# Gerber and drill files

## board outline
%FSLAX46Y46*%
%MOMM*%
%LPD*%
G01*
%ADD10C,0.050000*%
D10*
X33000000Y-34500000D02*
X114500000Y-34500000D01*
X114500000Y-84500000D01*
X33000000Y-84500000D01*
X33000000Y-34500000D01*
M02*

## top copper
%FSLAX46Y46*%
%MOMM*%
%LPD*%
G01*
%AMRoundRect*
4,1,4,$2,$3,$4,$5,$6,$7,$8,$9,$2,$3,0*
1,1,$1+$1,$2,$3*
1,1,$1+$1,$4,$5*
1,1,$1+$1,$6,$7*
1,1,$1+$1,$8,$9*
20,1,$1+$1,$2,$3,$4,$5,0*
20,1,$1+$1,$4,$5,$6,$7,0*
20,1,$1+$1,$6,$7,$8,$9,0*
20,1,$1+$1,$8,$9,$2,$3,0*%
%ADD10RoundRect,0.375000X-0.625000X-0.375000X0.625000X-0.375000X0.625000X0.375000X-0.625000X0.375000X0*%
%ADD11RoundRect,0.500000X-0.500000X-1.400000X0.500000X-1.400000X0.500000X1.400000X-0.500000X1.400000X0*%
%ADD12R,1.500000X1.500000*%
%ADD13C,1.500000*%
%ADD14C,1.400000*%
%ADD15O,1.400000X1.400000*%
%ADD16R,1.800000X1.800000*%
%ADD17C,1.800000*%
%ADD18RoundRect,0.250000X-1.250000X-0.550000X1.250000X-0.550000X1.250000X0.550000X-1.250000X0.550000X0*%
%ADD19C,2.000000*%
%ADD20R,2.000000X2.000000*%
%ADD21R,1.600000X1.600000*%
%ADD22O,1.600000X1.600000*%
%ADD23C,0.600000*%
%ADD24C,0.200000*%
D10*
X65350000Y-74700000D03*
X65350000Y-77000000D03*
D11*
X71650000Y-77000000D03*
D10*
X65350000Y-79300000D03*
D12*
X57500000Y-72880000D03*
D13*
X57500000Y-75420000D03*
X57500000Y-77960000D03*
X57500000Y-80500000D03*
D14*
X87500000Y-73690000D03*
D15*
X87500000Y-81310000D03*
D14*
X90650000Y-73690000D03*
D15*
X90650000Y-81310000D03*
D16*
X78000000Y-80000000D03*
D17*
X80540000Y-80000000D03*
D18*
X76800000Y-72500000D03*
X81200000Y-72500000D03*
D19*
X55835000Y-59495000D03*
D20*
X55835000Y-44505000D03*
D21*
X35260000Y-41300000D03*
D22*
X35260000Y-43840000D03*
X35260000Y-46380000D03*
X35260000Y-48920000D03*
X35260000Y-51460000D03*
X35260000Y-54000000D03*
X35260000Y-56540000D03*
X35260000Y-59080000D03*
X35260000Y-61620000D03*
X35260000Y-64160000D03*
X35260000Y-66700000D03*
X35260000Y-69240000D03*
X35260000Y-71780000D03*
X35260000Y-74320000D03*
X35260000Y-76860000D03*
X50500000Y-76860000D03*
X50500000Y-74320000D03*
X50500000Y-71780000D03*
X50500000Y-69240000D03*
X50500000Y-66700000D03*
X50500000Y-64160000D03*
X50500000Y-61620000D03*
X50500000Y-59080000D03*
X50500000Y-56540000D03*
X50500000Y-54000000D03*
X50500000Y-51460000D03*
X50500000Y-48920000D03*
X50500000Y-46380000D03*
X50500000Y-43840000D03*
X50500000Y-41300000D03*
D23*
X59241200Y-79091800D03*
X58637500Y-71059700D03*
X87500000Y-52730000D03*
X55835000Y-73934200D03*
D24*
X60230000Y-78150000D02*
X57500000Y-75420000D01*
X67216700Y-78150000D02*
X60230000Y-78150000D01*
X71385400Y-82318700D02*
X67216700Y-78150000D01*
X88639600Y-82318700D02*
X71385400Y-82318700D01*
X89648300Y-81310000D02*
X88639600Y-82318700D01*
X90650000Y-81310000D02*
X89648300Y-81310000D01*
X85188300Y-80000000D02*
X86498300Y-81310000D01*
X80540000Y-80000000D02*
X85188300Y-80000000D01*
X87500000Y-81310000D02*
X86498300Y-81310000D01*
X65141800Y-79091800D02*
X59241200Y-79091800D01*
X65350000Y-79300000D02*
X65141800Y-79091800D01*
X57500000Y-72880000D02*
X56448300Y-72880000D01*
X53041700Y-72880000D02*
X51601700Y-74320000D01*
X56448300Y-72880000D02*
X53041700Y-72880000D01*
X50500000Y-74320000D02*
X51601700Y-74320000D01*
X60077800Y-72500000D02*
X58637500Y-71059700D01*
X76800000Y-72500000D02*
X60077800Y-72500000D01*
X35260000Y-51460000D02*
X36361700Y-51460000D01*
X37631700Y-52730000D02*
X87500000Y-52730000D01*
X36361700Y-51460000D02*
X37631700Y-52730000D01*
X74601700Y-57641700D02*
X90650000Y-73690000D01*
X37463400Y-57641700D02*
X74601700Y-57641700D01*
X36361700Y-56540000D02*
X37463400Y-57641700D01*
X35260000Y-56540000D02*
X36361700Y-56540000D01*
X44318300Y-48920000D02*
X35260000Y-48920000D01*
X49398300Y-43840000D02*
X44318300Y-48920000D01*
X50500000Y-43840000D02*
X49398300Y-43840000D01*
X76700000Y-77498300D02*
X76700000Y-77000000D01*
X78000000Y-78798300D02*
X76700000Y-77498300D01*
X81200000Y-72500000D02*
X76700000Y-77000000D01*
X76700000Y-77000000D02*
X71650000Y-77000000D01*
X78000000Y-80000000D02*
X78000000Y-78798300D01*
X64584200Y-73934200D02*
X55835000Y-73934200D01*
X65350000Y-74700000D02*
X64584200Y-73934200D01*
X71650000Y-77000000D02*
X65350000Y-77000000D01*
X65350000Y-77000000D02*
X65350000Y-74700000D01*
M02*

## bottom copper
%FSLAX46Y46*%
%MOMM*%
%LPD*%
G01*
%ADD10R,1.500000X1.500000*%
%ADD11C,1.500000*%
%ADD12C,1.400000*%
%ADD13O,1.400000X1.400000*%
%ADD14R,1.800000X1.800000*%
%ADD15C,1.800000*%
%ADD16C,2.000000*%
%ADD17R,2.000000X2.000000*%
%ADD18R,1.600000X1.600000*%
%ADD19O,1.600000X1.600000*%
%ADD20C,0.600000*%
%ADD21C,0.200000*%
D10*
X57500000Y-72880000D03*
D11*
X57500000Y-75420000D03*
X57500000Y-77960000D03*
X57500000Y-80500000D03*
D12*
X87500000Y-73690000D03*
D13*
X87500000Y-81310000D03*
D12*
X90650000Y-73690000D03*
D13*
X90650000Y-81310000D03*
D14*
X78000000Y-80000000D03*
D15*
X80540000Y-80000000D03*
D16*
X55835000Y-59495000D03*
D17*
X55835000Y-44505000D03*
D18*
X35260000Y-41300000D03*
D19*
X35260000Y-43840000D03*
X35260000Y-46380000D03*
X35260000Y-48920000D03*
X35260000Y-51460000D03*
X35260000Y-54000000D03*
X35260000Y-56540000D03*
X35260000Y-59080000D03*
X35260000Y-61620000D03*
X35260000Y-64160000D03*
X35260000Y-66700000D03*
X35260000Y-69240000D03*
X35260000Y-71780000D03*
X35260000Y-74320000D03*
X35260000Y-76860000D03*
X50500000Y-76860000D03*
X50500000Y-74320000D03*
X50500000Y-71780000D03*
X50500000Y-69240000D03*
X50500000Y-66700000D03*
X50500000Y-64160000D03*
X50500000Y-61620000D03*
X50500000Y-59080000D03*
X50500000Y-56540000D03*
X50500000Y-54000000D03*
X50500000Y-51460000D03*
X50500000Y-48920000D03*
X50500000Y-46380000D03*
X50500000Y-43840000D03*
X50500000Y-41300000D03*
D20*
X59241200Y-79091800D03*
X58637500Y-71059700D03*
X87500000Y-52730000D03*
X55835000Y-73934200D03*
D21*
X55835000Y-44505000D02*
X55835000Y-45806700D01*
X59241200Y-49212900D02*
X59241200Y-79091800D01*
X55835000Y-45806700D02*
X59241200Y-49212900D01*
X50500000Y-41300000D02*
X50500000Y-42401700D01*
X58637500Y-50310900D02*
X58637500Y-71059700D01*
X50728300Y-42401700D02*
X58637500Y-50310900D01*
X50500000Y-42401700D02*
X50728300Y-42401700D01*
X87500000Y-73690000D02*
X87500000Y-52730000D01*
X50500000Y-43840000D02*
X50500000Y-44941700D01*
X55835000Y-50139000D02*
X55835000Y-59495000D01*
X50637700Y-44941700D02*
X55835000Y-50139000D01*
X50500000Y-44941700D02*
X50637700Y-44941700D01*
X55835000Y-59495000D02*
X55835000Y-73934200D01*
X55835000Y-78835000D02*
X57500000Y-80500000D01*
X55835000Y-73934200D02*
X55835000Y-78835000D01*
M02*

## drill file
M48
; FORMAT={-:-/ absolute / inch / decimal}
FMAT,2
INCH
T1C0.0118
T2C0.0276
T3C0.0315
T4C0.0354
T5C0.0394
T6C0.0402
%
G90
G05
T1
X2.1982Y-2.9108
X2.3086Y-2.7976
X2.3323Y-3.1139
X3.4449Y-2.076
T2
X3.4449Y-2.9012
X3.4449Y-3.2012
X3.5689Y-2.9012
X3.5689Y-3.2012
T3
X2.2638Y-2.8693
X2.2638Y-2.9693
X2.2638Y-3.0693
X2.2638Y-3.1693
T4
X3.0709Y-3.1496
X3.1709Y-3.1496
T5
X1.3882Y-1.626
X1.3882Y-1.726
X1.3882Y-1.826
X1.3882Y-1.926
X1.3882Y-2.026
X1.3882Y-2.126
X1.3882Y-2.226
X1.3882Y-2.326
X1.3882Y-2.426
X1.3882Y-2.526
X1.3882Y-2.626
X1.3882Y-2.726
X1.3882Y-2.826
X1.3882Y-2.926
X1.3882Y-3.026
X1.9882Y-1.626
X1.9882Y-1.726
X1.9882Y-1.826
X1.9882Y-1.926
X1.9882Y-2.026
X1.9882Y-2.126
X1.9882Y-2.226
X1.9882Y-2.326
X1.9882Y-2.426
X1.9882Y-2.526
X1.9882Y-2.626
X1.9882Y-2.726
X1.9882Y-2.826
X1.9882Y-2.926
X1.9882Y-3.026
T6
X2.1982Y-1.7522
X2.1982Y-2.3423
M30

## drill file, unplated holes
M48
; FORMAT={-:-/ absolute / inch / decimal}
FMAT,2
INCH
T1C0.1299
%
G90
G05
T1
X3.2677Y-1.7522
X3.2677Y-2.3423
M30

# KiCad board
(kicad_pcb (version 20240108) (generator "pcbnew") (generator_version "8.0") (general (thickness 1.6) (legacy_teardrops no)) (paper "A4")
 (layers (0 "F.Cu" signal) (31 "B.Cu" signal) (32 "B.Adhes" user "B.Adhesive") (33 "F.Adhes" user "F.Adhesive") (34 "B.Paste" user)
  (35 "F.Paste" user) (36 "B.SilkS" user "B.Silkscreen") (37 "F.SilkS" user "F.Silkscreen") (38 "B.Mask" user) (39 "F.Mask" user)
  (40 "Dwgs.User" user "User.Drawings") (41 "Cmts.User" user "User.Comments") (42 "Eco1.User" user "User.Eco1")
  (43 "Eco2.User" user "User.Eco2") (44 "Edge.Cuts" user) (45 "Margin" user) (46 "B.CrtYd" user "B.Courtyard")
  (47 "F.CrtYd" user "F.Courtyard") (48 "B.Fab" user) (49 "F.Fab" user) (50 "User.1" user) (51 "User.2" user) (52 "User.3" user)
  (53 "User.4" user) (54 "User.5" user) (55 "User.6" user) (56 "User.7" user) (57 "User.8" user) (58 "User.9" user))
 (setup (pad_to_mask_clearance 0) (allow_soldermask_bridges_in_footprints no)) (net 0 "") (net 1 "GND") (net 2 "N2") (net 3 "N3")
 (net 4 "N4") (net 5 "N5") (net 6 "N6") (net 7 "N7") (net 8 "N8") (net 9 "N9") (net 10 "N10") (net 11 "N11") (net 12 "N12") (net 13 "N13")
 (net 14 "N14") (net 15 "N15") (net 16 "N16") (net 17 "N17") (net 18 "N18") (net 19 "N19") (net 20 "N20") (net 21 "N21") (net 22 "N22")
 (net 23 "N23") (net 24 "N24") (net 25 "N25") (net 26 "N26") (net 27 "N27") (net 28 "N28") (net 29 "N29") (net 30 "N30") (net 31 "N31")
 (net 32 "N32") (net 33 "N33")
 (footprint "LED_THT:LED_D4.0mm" (layer "F.Cu") (at 78 80)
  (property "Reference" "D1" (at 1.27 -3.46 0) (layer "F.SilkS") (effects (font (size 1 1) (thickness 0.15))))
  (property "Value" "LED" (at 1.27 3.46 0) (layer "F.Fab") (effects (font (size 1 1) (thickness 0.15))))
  (pad "1" thru_hole rect (at 0 0) (size 1.8 1.8) (drill 0.9) (layers "*.Cu" "*.Mask") (remove_unused_layers no) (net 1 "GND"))
  (pad "2" thru_hole circle (at 2.54 0) (size 1.8 1.8) (drill 0.9) (layers "*.Cu" "*.Mask") (remove_unused_layers no) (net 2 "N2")))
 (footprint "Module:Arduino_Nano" (layer "F.Cu") (at 35.26 41.3)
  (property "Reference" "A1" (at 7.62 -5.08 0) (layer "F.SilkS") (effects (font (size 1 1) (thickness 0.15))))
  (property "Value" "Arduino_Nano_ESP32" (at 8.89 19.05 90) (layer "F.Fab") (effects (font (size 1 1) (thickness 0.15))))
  (pad "1" thru_hole rect (at 0 0) (size 1.6 1.6) (drill 1) (layers "*.Cu" "*.Mask") (remove_unused_layers no) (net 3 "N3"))
  (pad "2" thru_hole oval (at 0 2.54) (size 1.6 1.6) (drill 1) (layers "*.Cu" "*.Mask") (remove_unused_layers no) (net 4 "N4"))
  (pad "3" thru_hole oval (at 0 5.08) (size 1.6 1.6) (drill 1) (layers "*.Cu" "*.Mask") (remove_unused_layers no) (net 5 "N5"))
  (pad "4" thru_hole oval (at 0 7.62) (size 1.6 1.6) (drill 1) (layers "*.Cu" "*.Mask") (remove_unused_layers no) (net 1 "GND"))
  (pad "5" thru_hole oval (at 0 10.16) (size 1.6 1.6) (drill 1) (layers "*.Cu" "*.Mask") (remove_unused_layers no) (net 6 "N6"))
  (pad "6" thru_hole oval (at 0 12.7) (size 1.6 1.6) (drill 1) (layers "*.Cu" "*.Mask") (remove_unused_layers no) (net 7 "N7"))
  (pad "7" thru_hole oval (at 0 15.24) (size 1.6 1.6) (drill 1) (layers "*.Cu" "*.Mask") (remove_unused_layers no) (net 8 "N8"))
  (pad "8" thru_hole oval (at 0 17.78) (size 1.6 1.6) (drill 1) (layers "*.Cu" "*.Mask") (remove_unused_layers no) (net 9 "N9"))
  (pad "9" thru_hole oval (at 0 20.32) (size 1.6 1.6) (drill 1) (layers "*.Cu" "*.Mask") (remove_unused_layers no) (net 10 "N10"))
  (pad "10" thru_hole oval (at 0 22.86) (size 1.6 1.6) (drill 1) (layers "*.Cu" "*.Mask") (remove_unused_layers no) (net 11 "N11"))
  (pad "11" thru_hole oval (at 0 25.4) (size 1.6 1.6) (drill 1) (layers "*.Cu" "*.Mask") (remove_unused_layers no) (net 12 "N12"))
  (pad "12" thru_hole oval (at 0 27.94) (size 1.6 1.6) (drill 1) (layers "*.Cu" "*.Mask") (remove_unused_layers no) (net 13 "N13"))
  (pad "13" thru_hole oval (at 0 30.48) (size 1.6 1.6) (drill 1) (layers "*.Cu" "*.Mask") (remove_unused_layers no) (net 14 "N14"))
  (pad "14" thru_hole oval (at 0 33.02) (size 1.6 1.6) (drill 1) (layers "*.Cu" "*.Mask") (remove_unused_layers no) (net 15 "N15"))
  (pad "15" thru_hole oval (at 0 35.56) (size 1.6 1.6) (drill 1) (layers "*.Cu" "*.Mask") (remove_unused_layers no) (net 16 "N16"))
  (pad "16" thru_hole oval (at 15.24 35.56) (size 1.6 1.6) (drill 1) (layers "*.Cu" "*.Mask") (remove_unused_layers no) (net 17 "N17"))
  (pad "17" thru_hole oval (at 15.24 33.02) (size 1.6 1.6) (drill 1) (layers "*.Cu" "*.Mask") (remove_unused_layers no) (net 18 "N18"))
  (pad "18" thru_hole oval (at 15.24 30.48) (size 1.6 1.6) (drill 1) (layers "*.Cu" "*.Mask") (remove_unused_layers no) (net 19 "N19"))
  (pad "19" thru_hole oval (at 15.24 27.94) (size 1.6 1.6) (drill 1) (layers "*.Cu" "*.Mask") (remove_unused_layers no) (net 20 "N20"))
  (pad "20" thru_hole oval (at 15.24 25.4) (size 1.6 1.6) (drill 1) (layers "*.Cu" "*.Mask") (remove_unused_layers no) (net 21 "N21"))
  (pad "21" thru_hole oval (at 15.24 22.86) (size 1.6 1.6) (drill 1) (layers "*.Cu" "*.Mask") (remove_unused_layers no) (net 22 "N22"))
  (pad "22" thru_hole oval (at 15.24 20.32) (size 1.6 1.6) (drill 1) (layers "*.Cu" "*.Mask") (remove_unused_layers no) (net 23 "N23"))
  (pad "23" thru_hole oval (at 15.24 17.78) (size 1.6 1.6) (drill 1) (layers "*.Cu" "*.Mask") (remove_unused_layers no) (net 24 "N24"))
  (pad "24" thru_hole oval (at 15.24 15.24) (size 1.6 1.6) (drill 1) (layers "*.Cu" "*.Mask") (remove_unused_layers no) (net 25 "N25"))
  (pad "25" thru_hole oval (at 15.24 12.7) (size 1.6 1.6) (drill 1) (layers "*.Cu" "*.Mask") (remove_unused_layers no) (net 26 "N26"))
  (pad "26" thru_hole oval (at 15.24 10.16) (size 1.6 1.6) (drill 1) (layers "*.Cu" "*.Mask") (remove_unused_layers no) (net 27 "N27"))
  (pad "27" thru_hole oval (at 15.24 7.62) (size 1.6 1.6) (drill 1) (layers "*.Cu" "*.Mask") (remove_unused_layers no) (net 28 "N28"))
  (pad "28" thru_hole oval (at 15.24 5.08) (size 1.6 1.6) (drill 1) (layers "*.Cu" "*.Mask") (remove_unused_layers no) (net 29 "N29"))
  (pad "29" thru_hole oval (at 15.24 2.54) (size 1.6 1.6) (drill 1) (layers "*.Cu" "*.Mask") (remove_unused_layers no) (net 1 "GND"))
  (pad "30" thru_hole oval (at 15.24 0) (size 1.6 1.6) (drill 1) (layers "*.Cu" "*.Mask") (remove_unused_layers no) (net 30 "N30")))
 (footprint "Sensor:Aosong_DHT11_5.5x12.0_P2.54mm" (layer "F.Cu") (at 57.5 72.88)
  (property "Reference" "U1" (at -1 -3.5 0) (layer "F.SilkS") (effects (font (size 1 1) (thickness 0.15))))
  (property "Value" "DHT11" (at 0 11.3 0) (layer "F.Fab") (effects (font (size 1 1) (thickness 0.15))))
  (pad "1" thru_hole rect (at 0 0) (size 1.5 1.5) (drill 0.8) (layers "*.Cu" "*.Mask") (remove_unused_layers no) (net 18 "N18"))
  (pad "2" thru_hole circle (at 0 2.54) (size 1.5 1.5) (drill 0.8) (layers "*.Cu" "*.Mask") (remove_unused_layers no) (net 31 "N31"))
  (pad "3" thru_hole circle (at 0 5.08) (size 1.5 1.5) (drill 0.8) (layers "*.Cu" "*.Mask") (remove_unused_layers no) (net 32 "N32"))
  (pad "4" thru_hole circle (at 0 7.62) (size 1.5 1.5) (drill 0.8) (layers "*.Cu" "*.Mask") (remove_unused_layers no) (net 1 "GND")))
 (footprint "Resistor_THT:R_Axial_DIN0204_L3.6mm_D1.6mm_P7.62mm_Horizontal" (layer "F.Cu") (at 87.5 73.69 -90)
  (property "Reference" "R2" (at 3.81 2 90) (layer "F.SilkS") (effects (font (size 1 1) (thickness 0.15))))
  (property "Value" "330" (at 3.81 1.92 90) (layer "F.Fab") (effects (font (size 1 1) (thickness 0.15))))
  (pad "1" thru_hole circle (at 0 0 270) (size 1.4 1.4) (drill 0.7) (layers "*.Cu" "*.Mask") (remove_unused_layers no) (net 6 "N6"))
  (pad "2" thru_hole oval (at 7.62 0 270) (size 1.4 1.4) (drill 0.7) (layers "*.Cu" "*.Mask") (remove_unused_layers no) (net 2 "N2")))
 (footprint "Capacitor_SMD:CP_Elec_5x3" (layer "F.Cu") (at 79 72.5)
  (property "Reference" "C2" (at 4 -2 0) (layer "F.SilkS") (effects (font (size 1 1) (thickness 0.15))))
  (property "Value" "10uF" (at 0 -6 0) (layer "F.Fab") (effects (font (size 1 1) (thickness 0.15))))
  (pad "1" smd roundrect (at -2.2 0) (size 3 1.6) (layers "F.Cu" "F.Paste" "F.Mask") (roundrect_rratio 0.15625) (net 30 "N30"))
  (pad "2" smd roundrect (at 2.2 0) (size 3 1.6) (layers "F.Cu" "F.Paste" "F.Mask") (roundrect_rratio 0.15625) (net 1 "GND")))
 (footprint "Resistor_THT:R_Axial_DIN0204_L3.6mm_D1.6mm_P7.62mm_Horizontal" (layer "F.Cu") (at 90.65 73.69 -90)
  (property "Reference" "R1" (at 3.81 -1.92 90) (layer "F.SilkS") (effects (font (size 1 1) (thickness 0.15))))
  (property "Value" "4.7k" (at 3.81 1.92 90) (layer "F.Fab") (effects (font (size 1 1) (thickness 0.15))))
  (pad "1" thru_hole circle (at 0 0 270) (size 1.4 1.4) (drill 0.7) (layers "*.Cu" "*.Mask") (remove_unused_layers no) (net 8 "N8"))
  (pad "2" thru_hole oval (at 7.62 0 270) (size 1.4 1.4) (drill 0.7) (layers "*.Cu" "*.Mask") (remove_unused_layers no) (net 31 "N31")))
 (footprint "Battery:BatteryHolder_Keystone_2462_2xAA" (layer "F.Cu") (at 55.835 44.505)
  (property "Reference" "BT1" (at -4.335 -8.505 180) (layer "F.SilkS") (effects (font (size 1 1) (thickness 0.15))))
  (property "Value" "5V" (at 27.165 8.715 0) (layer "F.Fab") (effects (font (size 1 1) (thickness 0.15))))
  (pad "" np_thru_hole circle (at 27.165 0) (size 3.3 3.3) (drill 3.3) (layers "*.Cu" "*.Mask"))
  (pad "" np_thru_hole circle (at 27.165 14.99) (size 3.3 3.3) (drill 3.3) (layers "*.Cu" "*.Mask"))
  (pad "1" thru_hole rect (at 0 0) (size 2 2) (drill 1.02) (layers "*.Cu" "*.Mask") (remove_unused_layers no) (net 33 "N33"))
  (pad "2" thru_hole circle (at 0 14.99) (size 2 2) (drill 1.02) (layers "*.Cu" "*.Mask") (remove_unused_layers no) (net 1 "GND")))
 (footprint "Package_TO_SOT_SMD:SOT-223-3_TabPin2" (layer "F.Cu") (at 68.5 77)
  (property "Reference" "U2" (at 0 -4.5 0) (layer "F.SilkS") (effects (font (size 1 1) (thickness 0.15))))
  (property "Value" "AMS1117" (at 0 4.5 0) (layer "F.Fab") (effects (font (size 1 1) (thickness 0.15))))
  (pad "1" smd roundrect (at -3.15 -2.3) (size 2 1.5) (layers "F.Cu" "F.Paste" "F.Mask") (roundrect_rratio 0.25) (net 1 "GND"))
  (pad "2" smd roundrect (at -3.15 0) (size 2 1.5) (layers "F.Cu" "F.Paste" "F.Mask") (roundrect_rratio 0.25) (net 1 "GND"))
  (pad "2" smd roundrect (at 3.15 0) (size 2 3.8) (layers "F.Cu" "F.Paste" "F.Mask") (roundrect_rratio 0.25) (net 1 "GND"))
  (pad "3" smd roundrect (at -3.15 2.3) (size 2 1.5) (layers "F.Cu" "F.Paste" "F.Mask") (roundrect_rratio 0.25) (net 33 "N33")))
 (gr_rect (start 33 34.5) (end 114.5 84.5) (locked yes) (stroke (width 0.05) (type default)) (fill none) (layer "Edge.Cuts"))
 (segment (start 81.2 72.5) (end 76.7 77) (width 0.2) (layer "F.Cu") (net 1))
 (segment (start 76.7 77) (end 71.65 77) (width 0.2) (layer "F.Cu") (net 1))
 (segment (start 76.7 77.4983) (end 76.7 77) (width 0.2) (layer "F.Cu") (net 1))
 (segment (start 71.65 77) (end 65.35 77) (width 0.2) (layer "F.Cu") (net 1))
 (segment (start 64.5842 73.9342) (end 55.835 73.9342) (width 0.2) (layer "F.Cu") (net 1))
 (segment (start 50.5 43.84) (end 49.3983 43.84) (width 0.2) (layer "F.Cu") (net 1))
 (segment (start 78 80) (end 78 78.7983) (width 0.2) (layer "F.Cu") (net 1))
 (segment (start 49.3983 43.84) (end 44.3183 48.92) (width 0.2) (layer "F.Cu") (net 1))
 (segment (start 44.3183 48.92) (end 35.26 48.92) (width 0.2) (layer "F.Cu") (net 1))
 (segment (start 78 78.7983) (end 76.7 77.4983) (width 0.2) (layer "F.Cu") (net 1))
 (segment (start 65.35 77) (end 65.35 74.7) (width 0.2) (layer "F.Cu") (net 1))
 (segment (start 65.35 74.7) (end 64.5842 73.9342) (width 0.2) (layer "F.Cu") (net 1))
 (via (at 55.835 73.9342) (size 0.6) (drill 0.3) (layers "F.Cu" "B.Cu") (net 1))
 (segment (start 55.835 50.139) (end 55.835 59.495) (width 0.2) (layer "B.Cu") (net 1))
 (segment (start 55.835 73.9342) (end 55.835 78.835) (width 0.2) (layer "B.Cu") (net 1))
 (segment (start 50.5 43.84) (end 50.5 44.9417) (width 0.2) (layer "B.Cu") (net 1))
 (segment (start 50.5 44.9417) (end 50.6377 44.9417) (width 0.2) (layer "B.Cu") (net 1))
 (segment (start 55.835 59.495) (end 55.835 73.9342) (width 0.2) (layer "B.Cu") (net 1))
 (segment (start 55.835 78.835) (end 57.5 80.5) (width 0.2) (layer "B.Cu") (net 1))
 (segment (start 50.6377 44.9417) (end 55.835 50.139) (width 0.2) (layer "B.Cu") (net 1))
 (segment (start 35.26 56.54) (end 36.3617 56.54) (width 0.2) (layer "F.Cu") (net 8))
 (segment (start 36.3617 56.54) (end 37.4634 57.6417) (width 0.2) (layer "F.Cu") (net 8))
 (segment (start 74.6017 57.6417) (end 90.65 73.69) (width 0.2) (layer "F.Cu") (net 8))
 (segment (start 37.4634 57.6417) (end 74.6017 57.6417) (width 0.2) (layer "F.Cu") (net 8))
 (segment (start 35.26 51.46) (end 36.3617 51.46) (width 0.2) (layer "F.Cu") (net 6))
 (segment (start 36.3617 51.46) (end 37.6317 52.73) (width 0.2) (layer "F.Cu") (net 6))
 (segment (start 37.6317 52.73) (end 87.5 52.73) (width 0.2) (layer "F.Cu") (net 6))
 (via (at 87.5 52.73) (size 0.6) (drill 0.3) (layers "F.Cu" "B.Cu") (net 6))
 (segment (start 87.5 73.69) (end 87.5 52.73) (width 0.2) (layer "B.Cu") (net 6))
 (segment (start 60.0778 72.5) (end 58.6375 71.0597) (width 0.2) (layer "F.Cu") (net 30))
 (segment (start 76.8 72.5) (end 60.0778 72.5) (width 0.2) (layer "F.Cu") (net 30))
 (via (at 58.6375 71.0597) (size 0.6) (drill 0.3) (layers "F.Cu" "B.Cu") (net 30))
 (segment (start 50.5 41.3) (end 50.5 42.4017) (width 0.2) (layer "B.Cu") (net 30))
 (segment (start 58.6375 50.3109) (end 58.6375 71.0597) (width 0.2) (layer "B.Cu") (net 30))
 (segment (start 50.5 42.4017) (end 50.7283 42.4017) (width 0.2) (layer "B.Cu") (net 30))
 (segment (start 50.7283 42.4017) (end 58.6375 50.3109) (width 0.2) (layer "B.Cu") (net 30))
 (segment (start 57.5 72.88) (end 56.4483 72.88) (width 0.2) (layer "F.Cu") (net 18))
 (segment (start 53.0417 72.88) (end 51.6017 74.32) (width 0.2) (layer "F.Cu") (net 18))
 (segment (start 56.4483 72.88) (end 53.0417 72.88) (width 0.2) (layer "F.Cu") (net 18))
 (segment (start 50.5 74.32) (end 51.6017 74.32) (width 0.2) (layer "F.Cu") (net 18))
 (segment (start 65.1418 79.0918) (end 59.2412 79.0918) (width 0.2) (layer "F.Cu") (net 33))
 (segment (start 65.35 79.3) (end 65.1418 79.0918) (width 0.2) (layer "F.Cu") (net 33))
 (via (at 59.2412 79.0918) (size 0.6) (drill 0.3) (layers "F.Cu" "B.Cu") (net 33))
 (segment (start 55.835 45.8067) (end 59.2412 49.2129) (width 0.2) (layer "B.Cu") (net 33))
 (segment (start 55.835 44.505) (end 55.835 45.8067) (width 0.2) (layer "B.Cu") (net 33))
 (segment (start 59.2412 49.2129) (end 59.2412 79.0918) (width 0.2) (layer "B.Cu") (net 33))
 (segment (start 87.5 81.31) (end 86.4983 81.31) (width 0.2) (layer "F.Cu") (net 2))
 (segment (start 85.1883 80) (end 86.4983 81.31) (width 0.2) (layer "F.Cu") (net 2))
 (segment (start 80.54 80) (end 85.1883 80) (width 0.2) (layer "F.Cu") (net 2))
 (segment (start 90.65 81.31) (end 89.6483 81.31) (width 0.2) (layer "F.Cu") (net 31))
 (segment (start 88.6396 82.3187) (end 71.3854 82.3187) (width 0.2) (layer "F.Cu") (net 31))
 (segment (start 71.3854 82.3187) (end 67.2167 78.15) (width 0.2) (layer "F.Cu") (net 31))
 (segment (start 60.23 78.15) (end 57.5 75.42) (width 0.2) (layer "F.Cu") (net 31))
 (segment (start 67.2167 78.15) (end 60.23 78.15) (width 0.2) (layer "F.Cu") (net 31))
 (segment (start 89.6483 81.31) (end 88.6396 82.3187) (width 0.2) (layer "F.Cu") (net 31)))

